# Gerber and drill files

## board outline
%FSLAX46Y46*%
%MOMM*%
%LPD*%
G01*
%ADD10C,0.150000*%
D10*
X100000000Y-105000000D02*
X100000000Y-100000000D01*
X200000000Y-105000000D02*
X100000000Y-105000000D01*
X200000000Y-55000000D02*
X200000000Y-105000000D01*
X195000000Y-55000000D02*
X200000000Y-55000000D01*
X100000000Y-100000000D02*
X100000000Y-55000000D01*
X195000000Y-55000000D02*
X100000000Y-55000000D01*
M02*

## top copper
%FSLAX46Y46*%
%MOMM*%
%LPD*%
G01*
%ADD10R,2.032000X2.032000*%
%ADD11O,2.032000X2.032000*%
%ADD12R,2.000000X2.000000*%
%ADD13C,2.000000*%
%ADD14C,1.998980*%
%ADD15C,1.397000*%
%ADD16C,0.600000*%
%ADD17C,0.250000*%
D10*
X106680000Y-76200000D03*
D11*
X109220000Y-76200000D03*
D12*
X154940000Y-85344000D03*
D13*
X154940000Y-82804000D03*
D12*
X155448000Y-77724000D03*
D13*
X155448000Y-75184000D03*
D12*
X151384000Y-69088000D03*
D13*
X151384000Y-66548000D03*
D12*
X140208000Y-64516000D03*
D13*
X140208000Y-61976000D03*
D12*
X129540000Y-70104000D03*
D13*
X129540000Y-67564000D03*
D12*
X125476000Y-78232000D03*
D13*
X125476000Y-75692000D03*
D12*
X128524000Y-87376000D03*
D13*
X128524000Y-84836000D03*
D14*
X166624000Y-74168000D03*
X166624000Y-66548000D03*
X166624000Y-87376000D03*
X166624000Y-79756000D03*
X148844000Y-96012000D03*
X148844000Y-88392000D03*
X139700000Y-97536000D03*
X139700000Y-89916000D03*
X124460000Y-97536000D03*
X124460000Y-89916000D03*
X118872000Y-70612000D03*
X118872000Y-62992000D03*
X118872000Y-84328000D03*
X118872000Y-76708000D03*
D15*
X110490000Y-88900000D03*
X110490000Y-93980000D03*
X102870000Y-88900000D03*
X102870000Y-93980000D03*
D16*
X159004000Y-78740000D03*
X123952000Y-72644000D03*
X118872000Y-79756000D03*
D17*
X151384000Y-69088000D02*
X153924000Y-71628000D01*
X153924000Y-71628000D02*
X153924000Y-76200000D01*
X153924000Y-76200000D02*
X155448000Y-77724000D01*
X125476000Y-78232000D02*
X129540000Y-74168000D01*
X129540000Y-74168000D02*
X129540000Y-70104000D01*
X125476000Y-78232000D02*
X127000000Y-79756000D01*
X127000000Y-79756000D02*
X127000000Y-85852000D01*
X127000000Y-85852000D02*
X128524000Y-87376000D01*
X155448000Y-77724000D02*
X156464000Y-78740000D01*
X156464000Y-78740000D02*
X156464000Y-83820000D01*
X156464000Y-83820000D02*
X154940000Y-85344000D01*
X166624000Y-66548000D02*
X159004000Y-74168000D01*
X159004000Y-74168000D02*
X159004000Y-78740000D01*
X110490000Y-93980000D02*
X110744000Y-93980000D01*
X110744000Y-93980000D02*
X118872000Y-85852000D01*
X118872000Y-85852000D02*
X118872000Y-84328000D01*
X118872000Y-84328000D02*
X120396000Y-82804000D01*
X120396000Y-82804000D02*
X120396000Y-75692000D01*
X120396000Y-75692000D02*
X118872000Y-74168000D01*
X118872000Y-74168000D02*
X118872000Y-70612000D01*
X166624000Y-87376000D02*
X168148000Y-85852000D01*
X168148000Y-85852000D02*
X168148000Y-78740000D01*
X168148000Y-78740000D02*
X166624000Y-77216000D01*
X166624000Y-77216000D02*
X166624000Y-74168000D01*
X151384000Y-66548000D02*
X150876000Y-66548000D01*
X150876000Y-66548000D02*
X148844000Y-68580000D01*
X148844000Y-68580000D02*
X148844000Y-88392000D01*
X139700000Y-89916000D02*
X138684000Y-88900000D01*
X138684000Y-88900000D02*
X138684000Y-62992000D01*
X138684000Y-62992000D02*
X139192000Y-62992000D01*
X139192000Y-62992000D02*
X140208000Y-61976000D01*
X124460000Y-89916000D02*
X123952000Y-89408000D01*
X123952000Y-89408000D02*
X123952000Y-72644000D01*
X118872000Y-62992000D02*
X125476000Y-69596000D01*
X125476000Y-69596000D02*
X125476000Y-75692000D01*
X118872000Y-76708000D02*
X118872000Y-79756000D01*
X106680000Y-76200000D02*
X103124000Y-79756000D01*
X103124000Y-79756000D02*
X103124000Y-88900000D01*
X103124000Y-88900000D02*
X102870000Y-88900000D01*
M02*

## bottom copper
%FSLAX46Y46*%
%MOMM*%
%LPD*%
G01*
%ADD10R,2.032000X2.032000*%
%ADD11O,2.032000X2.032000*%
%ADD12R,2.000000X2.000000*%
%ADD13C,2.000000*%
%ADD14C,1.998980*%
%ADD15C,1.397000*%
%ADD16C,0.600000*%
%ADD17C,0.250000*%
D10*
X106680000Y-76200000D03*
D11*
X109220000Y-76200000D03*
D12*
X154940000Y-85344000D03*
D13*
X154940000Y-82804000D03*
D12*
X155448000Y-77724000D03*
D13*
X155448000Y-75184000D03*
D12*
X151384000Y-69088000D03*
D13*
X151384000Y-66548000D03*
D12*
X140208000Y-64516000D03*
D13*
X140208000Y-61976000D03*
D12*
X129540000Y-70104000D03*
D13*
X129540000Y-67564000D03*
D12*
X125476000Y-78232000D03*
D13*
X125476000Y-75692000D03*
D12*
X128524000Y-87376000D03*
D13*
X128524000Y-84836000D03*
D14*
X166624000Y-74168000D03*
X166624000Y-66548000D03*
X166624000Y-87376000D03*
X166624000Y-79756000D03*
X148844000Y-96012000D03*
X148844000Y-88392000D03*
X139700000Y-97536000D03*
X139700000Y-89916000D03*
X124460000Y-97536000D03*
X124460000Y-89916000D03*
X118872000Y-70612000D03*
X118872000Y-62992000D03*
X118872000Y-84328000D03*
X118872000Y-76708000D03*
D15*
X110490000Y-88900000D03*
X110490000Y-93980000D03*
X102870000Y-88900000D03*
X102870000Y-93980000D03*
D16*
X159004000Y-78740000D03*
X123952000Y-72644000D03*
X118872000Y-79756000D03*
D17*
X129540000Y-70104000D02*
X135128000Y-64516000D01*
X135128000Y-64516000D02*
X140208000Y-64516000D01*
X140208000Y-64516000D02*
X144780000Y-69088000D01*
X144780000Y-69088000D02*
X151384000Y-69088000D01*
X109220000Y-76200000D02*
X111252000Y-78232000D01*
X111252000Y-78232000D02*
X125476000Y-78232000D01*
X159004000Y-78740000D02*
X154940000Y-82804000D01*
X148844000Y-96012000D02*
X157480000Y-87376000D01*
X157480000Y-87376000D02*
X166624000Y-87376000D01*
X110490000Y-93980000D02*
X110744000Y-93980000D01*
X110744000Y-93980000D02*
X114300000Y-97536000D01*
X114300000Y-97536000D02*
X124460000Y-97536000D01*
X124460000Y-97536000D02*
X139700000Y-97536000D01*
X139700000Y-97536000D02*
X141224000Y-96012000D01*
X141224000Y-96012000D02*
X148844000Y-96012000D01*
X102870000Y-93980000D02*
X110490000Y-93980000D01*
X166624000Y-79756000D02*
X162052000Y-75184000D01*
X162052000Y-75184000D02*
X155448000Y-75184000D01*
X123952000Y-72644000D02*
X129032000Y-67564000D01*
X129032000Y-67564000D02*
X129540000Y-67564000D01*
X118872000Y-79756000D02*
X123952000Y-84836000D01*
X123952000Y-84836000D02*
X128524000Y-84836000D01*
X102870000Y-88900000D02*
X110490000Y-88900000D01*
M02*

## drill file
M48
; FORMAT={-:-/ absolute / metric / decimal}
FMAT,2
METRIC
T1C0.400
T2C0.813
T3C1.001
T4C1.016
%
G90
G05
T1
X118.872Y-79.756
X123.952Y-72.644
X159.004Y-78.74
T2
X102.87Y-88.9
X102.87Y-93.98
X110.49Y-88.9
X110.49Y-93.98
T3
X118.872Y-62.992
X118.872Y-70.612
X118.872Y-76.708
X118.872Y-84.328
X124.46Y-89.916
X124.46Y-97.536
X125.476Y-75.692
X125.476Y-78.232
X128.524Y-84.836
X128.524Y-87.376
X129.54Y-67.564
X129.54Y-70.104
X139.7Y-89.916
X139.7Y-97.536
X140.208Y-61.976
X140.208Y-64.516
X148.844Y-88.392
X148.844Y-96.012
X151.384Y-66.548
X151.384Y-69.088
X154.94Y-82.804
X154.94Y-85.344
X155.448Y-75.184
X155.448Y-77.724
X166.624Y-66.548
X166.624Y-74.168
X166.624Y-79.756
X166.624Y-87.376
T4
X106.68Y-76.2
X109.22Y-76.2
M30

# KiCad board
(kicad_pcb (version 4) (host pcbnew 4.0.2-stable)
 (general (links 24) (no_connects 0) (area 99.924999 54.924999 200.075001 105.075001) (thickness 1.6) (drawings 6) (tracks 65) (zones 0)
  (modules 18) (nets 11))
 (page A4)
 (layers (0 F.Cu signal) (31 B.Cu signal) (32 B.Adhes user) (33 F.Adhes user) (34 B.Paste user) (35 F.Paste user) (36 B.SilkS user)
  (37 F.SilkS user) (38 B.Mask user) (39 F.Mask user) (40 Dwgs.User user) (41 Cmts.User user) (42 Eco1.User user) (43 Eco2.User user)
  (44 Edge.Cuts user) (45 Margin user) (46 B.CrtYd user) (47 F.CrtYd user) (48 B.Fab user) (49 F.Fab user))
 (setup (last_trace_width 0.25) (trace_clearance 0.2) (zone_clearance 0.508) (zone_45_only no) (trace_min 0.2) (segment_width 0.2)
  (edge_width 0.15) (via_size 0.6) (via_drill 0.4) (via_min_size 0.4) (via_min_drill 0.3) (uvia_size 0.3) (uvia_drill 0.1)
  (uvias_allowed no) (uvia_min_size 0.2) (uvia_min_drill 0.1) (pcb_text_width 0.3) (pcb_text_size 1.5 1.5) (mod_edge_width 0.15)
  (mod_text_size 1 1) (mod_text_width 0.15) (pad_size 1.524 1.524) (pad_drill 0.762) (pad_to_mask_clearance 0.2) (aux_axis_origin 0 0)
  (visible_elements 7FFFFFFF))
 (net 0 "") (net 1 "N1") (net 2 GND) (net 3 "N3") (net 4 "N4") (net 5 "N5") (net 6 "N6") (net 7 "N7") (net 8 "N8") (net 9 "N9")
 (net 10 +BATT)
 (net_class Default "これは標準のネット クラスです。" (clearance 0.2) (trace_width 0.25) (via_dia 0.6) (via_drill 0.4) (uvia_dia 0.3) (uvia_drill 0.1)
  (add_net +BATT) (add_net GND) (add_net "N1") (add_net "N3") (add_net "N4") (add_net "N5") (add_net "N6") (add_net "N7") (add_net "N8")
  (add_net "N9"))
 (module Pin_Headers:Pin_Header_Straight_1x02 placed (layer F.Cu) (at 106.68 76.2 90)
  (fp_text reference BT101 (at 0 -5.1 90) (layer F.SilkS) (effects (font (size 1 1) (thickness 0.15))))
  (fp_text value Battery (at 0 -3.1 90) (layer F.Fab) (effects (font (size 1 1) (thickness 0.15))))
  (pad 1 thru_hole rect (at 0 0 90) (size 2.032 2.032) (drill 1.016) (layers *.Cu *.Mask F.SilkS) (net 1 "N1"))
  (pad 2 thru_hole oval (at 0 2.54 90) (size 2.032 2.032) (drill 1.016) (layers *.Cu *.Mask F.SilkS) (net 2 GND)))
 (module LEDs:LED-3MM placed (layer F.Cu) (at 154.94 85.344 90)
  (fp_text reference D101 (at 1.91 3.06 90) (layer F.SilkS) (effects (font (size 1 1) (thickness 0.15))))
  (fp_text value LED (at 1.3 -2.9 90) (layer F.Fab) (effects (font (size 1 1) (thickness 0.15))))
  (pad 1 thru_hole rect (at 0 0 180) (size 2 2) (drill 1.00076) (layers *.Cu *.Mask F.SilkS) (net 2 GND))
  (pad 2 thru_hole circle (at 2.54 0 90) (size 2 2) (drill 1.00076) (layers *.Cu *.Mask F.SilkS) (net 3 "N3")))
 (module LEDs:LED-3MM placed (layer F.Cu) (at 155.448 77.724 90)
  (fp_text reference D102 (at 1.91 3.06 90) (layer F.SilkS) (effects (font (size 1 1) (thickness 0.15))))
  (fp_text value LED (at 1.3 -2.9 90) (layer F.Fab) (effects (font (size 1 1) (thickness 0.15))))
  (pad 1 thru_hole rect (at 0 0 180) (size 2 2) (drill 1.00076) (layers *.Cu *.Mask F.SilkS) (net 2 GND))
  (pad 2 thru_hole circle (at 2.54 0 90) (size 2 2) (drill 1.00076) (layers *.Cu *.Mask F.SilkS) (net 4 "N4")))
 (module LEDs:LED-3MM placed (layer F.Cu) (at 151.384 69.088 90)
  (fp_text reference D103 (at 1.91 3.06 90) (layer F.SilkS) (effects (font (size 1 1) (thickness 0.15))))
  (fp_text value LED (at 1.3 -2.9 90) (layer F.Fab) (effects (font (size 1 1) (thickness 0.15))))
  (pad 1 thru_hole rect (at 0 0 180) (size 2 2) (drill 1.00076) (layers *.Cu *.Mask F.SilkS) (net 2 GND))
  (pad 2 thru_hole circle (at 2.54 0 90) (size 2 2) (drill 1.00076) (layers *.Cu *.Mask F.SilkS) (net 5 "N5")))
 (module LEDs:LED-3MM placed (layer F.Cu) (at 140.208 64.516 90)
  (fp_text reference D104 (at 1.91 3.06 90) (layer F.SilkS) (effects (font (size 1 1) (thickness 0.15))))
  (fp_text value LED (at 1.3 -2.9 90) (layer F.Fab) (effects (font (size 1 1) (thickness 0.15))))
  (pad 1 thru_hole rect (at 0 0 180) (size 2 2) (drill 1.00076) (layers *.Cu *.Mask F.SilkS) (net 2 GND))
  (pad 2 thru_hole circle (at 2.54 0 90) (size 2 2) (drill 1.00076) (layers *.Cu *.Mask F.SilkS) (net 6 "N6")))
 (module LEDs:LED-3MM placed (layer F.Cu) (at 129.54 70.104 90)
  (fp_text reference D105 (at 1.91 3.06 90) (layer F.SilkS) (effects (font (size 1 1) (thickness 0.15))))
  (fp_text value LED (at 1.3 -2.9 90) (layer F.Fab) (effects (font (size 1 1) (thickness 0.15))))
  (pad 1 thru_hole rect (at 0 0 180) (size 2 2) (drill 1.00076) (layers *.Cu *.Mask F.SilkS) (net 2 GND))
  (pad 2 thru_hole circle (at 2.54 0 90) (size 2 2) (drill 1.00076) (layers *.Cu *.Mask F.SilkS) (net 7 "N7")))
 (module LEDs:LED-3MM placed (layer F.Cu) (at 125.476 78.232 90)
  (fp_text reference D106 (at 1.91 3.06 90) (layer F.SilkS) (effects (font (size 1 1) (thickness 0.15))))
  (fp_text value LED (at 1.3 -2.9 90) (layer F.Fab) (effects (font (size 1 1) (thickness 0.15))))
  (pad 1 thru_hole rect (at 0 0 180) (size 2 2) (drill 1.00076) (layers *.Cu *.Mask F.SilkS) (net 2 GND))
  (pad 2 thru_hole circle (at 2.54 0 90) (size 2 2) (drill 1.00076) (layers *.Cu *.Mask F.SilkS) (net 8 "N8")))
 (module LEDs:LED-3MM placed (layer F.Cu) (at 128.524 87.376 90)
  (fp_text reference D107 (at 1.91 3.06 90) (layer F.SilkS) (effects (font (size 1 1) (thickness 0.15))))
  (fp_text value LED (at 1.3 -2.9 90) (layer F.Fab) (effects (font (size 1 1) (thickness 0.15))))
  (pad 1 thru_hole rect (at 0 0 180) (size 2 2) (drill 1.00076) (layers *.Cu *.Mask F.SilkS) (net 2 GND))
  (pad 2 thru_hole circle (at 2.54 0 90) (size 2 2) (drill 1.00076) (layers *.Cu *.Mask F.SilkS) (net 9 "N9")))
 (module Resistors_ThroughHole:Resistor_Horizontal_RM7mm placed (layer F.Cu) (at 166.624 74.168 90)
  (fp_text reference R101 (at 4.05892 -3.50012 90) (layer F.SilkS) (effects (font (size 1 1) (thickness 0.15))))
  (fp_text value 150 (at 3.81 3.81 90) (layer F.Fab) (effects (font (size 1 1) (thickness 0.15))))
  (pad 1 thru_hole circle (at 0 0 90) (size 1.99898 1.99898) (drill 1.00076) (layers *.Cu *.SilkS *.Mask) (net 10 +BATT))
  (pad 2 thru_hole circle (at 7.62 0 90) (size 1.99898 1.99898) (drill 1.00076) (layers *.Cu *.SilkS *.Mask) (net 3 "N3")))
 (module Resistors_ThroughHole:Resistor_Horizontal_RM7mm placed (layer F.Cu) (at 166.624 87.376 90)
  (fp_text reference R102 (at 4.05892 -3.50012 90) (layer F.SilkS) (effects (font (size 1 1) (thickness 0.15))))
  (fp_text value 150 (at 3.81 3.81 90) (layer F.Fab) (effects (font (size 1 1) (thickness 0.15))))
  (pad 1 thru_hole circle (at 0 0 90) (size 1.99898 1.99898) (drill 1.00076) (layers *.Cu *.SilkS *.Mask) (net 10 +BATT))
  (pad 2 thru_hole circle (at 7.62 0 90) (size 1.99898 1.99898) (drill 1.00076) (layers *.Cu *.SilkS *.Mask) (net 4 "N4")))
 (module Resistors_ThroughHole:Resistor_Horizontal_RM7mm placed (layer F.Cu) (at 148.844 96.012 90)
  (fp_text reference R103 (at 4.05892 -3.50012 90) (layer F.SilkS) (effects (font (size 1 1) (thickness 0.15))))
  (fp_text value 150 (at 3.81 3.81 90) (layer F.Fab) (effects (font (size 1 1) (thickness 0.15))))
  (pad 1 thru_hole circle (at 0 0 90) (size 1.99898 1.99898) (drill 1.00076) (layers *.Cu *.SilkS *.Mask) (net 10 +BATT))
  (pad 2 thru_hole circle (at 7.62 0 90) (size 1.99898 1.99898) (drill 1.00076) (layers *.Cu *.SilkS *.Mask) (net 5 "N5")))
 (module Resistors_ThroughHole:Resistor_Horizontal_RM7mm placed (layer F.Cu) (at 139.7 97.536 90)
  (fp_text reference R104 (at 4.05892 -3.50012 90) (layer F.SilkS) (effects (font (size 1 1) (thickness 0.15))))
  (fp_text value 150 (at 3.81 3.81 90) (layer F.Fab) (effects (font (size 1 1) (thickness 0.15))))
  (pad 1 thru_hole circle (at 0 0 90) (size 1.99898 1.99898) (drill 1.00076) (layers *.Cu *.SilkS *.Mask) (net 10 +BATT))
  (pad 2 thru_hole circle (at 7.62 0 90) (size 1.99898 1.99898) (drill 1.00076) (layers *.Cu *.SilkS *.Mask) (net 6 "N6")))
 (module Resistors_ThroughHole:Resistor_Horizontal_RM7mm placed (layer F.Cu) (at 124.46 97.536 90)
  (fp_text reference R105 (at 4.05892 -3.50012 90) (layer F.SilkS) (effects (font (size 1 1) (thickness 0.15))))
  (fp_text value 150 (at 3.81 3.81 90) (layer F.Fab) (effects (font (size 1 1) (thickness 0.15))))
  (pad 1 thru_hole circle (at 0 0 90) (size 1.99898 1.99898) (drill 1.00076) (layers *.Cu *.SilkS *.Mask) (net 10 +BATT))
  (pad 2 thru_hole circle (at 7.62 0 90) (size 1.99898 1.99898) (drill 1.00076) (layers *.Cu *.SilkS *.Mask) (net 7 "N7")))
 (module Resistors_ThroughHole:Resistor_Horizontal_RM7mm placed (layer F.Cu) (at 118.872 70.612 90)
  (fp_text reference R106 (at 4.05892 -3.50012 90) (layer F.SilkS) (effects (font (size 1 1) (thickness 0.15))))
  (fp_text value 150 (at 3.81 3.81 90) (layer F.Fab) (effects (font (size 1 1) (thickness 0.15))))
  (pad 1 thru_hole circle (at 0 0 90) (size 1.99898 1.99898) (drill 1.00076) (layers *.Cu *.SilkS *.Mask) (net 10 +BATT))
  (pad 2 thru_hole circle (at 7.62 0 90) (size 1.99898 1.99898) (drill 1.00076) (layers *.Cu *.SilkS *.Mask) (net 8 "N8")))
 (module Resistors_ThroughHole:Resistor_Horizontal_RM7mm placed (layer F.Cu) (at 118.872 84.328 90)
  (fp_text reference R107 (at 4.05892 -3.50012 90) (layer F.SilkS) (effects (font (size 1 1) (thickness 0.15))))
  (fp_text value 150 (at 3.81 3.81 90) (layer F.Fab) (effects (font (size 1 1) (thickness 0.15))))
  (pad 1 thru_hole circle (at 0 0 90) (size 1.99898 1.99898) (drill 1.00076) (layers *.Cu *.SilkS *.Mask) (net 10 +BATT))
  (pad 2 thru_hole circle (at 7.62 0 90) (size 1.99898 1.99898) (drill 1.00076) (layers *.Cu *.SilkS *.Mask) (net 9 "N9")))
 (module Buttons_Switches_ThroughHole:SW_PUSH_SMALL (layer F.Cu) (at 106.68 91.44)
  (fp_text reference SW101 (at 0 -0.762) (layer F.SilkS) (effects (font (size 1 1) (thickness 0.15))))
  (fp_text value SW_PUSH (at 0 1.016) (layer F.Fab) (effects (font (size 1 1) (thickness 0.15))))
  (pad 1 thru_hole circle (at 3.81 -2.54) (size 1.397 1.397) (drill 0.8128) (layers *.Cu *.Mask F.SilkS) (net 1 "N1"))
  (pad 2 thru_hole circle (at 3.81 2.54) (size 1.397 1.397) (drill 0.8128) (layers *.Cu *.Mask F.SilkS) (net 10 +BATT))
  (pad 1 thru_hole circle (at -3.81 -2.54) (size 1.397 1.397) (drill 0.8128) (layers *.Cu *.Mask F.SilkS) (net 1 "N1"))
  (pad 2 thru_hole circle (at -3.81 2.54) (size 1.397 1.397) (drill 0.8128) (layers *.Cu *.Mask F.SilkS) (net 10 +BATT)))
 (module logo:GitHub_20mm (layer F.Cu) (at 139.7 77.724)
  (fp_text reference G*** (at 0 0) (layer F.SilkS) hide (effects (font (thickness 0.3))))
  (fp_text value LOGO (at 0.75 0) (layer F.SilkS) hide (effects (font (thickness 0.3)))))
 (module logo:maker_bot (layer F.Cu) (at 181.864 75.692)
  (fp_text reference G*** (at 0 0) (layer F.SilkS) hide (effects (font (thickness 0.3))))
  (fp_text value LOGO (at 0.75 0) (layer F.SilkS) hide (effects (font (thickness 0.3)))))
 (gr_line (start 100 105) (end 100 100) (angle 90) (layer Edge.Cuts) (width 0.15))
 (gr_line (start 200 105) (end 100 105) (angle 90) (layer Edge.Cuts) (width 0.15))
 (gr_line (start 200 55) (end 200 105) (angle 90) (layer Edge.Cuts) (width 0.15))
 (gr_line (start 195 55) (end 200 55) (angle 90) (layer Edge.Cuts) (width 0.15))
 (gr_line (start 100 100) (end 100 55) (angle 90) (layer Edge.Cuts) (width 0.15))
 (gr_line (start 195 55) (end 100 55) (angle 90) (layer Edge.Cuts) (width 0.15))
 (segment (start 129.54 70.104) (end 135.128 64.516) (width 0.25) (layer B.Cu) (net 2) (status 80000))
 (segment (start 135.128 64.516) (end 140.208 64.516) (width 0.25) (layer B.Cu) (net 2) (status 80000))
 (segment (start 140.208 64.516) (end 144.78 69.088) (width 0.25) (layer B.Cu) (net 2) (status 80000))
 (segment (start 144.78 69.088) (end 151.384 69.088) (width 0.25) (layer B.Cu) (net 2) (status 80000))
 (segment (start 151.384 69.088) (end 153.924 71.628) (width 0.25) (layer F.Cu) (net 2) (status 80000))
 (segment (start 153.924 71.628) (end 153.924 76.2) (width 0.25) (layer F.Cu) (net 2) (status 80000))
 (segment (start 153.924 76.2) (end 155.448 77.724) (width 0.25) (layer F.Cu) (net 2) (status 80000))
 (segment (start 125.476 78.232) (end 129.54 74.168) (width 0.25) (layer F.Cu) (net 2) (status 80000))
 (segment (start 129.54 74.168) (end 129.54 70.104) (width 0.25) (layer F.Cu) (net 2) (status 80000))
 (segment (start 109.22 76.2) (end 111.252 78.232) (width 0.25) (layer B.Cu) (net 2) (status 80000))
 (segment (start 111.252 78.232) (end 125.476 78.232) (width 0.25) (layer B.Cu) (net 2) (status 80000))
 (segment (start 125.476 78.232) (end 127 79.756) (width 0.25) (layer F.Cu) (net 2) (status 80000))
 (segment (start 127 79.756) (end 127 85.852) (width 0.25) (layer F.Cu) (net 2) (status 80000))
 (segment (start 127 85.852) (end 128.524 87.376) (width 0.25) (layer F.Cu) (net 2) (status 80000))
 (segment (start 155.448 77.724) (end 156.464 78.74) (width 0.25) (layer F.Cu) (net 2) (status 80000))
 (segment (start 156.464 78.74) (end 156.464 83.82) (width 0.25) (layer F.Cu) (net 2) (status 80000))
 (segment (start 156.464 83.82) (end 154.94 85.344) (width 0.25) (layer F.Cu) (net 2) (status 80000))
 (segment (start 166.624 66.548) (end 159.004 74.168) (width 0.25) (layer F.Cu) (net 3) (status 80000))
 (segment (start 159.004 74.168) (end 159.004 78.74) (width 0.25) (layer F.Cu) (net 3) (status 80000))
 (via (at 159.004 78.74) (size 0.6) (layers F.Cu B.Cu) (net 3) (status 80000))
 (segment (start 159.004 78.74) (end 154.94 82.804) (width 0.25) (layer B.Cu) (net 3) (status 80000))
 (segment (start 148.844 96.012) (end 157.48 87.376) (width 0.25) (layer B.Cu) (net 10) (status 80000))
 (segment (start 157.48 87.376) (end 166.624 87.376) (width 0.25) (layer B.Cu) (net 10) (status 80000))
 (segment (start 110.49 93.98) (end 110.744 93.98) (width 0.25) (layer F.Cu) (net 10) (status 80000))
 (segment (start 110.744 93.98) (end 118.872 85.852) (width 0.25) (layer F.Cu) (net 10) (status 80000))
 (segment (start 118.872 85.852) (end 118.872 84.328) (width 0.25) (layer F.Cu) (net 10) (status 80000))
 (segment (start 110.49 93.98) (end 110.744 93.98) (width 0.25) (layer B.Cu) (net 10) (status 80000))
 (segment (start 110.744 93.98) (end 114.3 97.536) (width 0.25) (layer B.Cu) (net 10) (status 80000))
 (segment (start 114.3 97.536) (end 124.46 97.536) (width 0.25) (layer B.Cu) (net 10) (status 80000))
 (segment (start 124.46 97.536) (end 139.7 97.536) (width 0.25) (layer B.Cu) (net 10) (status 80000))
 (segment (start 139.7 97.536) (end 141.224 96.012) (width 0.25) (layer B.Cu) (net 10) (status 80000))
 (segment (start 141.224 96.012) (end 148.844 96.012) (width 0.25) (layer B.Cu) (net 10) (status 80000))
 (segment (start 118.872 84.328) (end 120.396 82.804) (width 0.25) (layer F.Cu) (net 10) (status 80000))
 (segment (start 120.396 82.804) (end 120.396 75.692) (width 0.25) (layer F.Cu) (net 10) (status 80000))
 (segment (start 120.396 75.692) (end 118.872 74.168) (width 0.25) (layer F.Cu) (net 10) (status 80000))
 (segment (start 118.872 74.168) (end 118.872 70.612) (width 0.25) (layer F.Cu) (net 10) (status 80000))
 (segment (start 166.624 87.376) (end 168.148 85.852) (width 0.25) (layer F.Cu) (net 10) (status 80000))
 (segment (start 168.148 85.852) (end 168.148 78.74) (width 0.25) (layer F.Cu) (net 10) (status 80000))
 (segment (start 168.148 78.74) (end 166.624 77.216) (width 0.25) (layer F.Cu) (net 10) (status 80000))
 (segment (start 166.624 77.216) (end 166.624 74.168) (width 0.25) (layer F.Cu) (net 10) (status 80000))
 (segment (start 102.87 93.98) (end 110.49 93.98) (width 0.25) (layer B.Cu) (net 10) (status 80000))
 (segment (start 166.624 79.756) (end 162.052 75.184) (width 0.25) (layer B.Cu) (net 4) (status 80000))
 (segment (start 162.052 75.184) (end 155.448 75.184) (width 0.25) (layer B.Cu) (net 4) (status 80000))
 (segment (start 151.384 66.548) (end 150.876 66.548) (width 0.25) (layer F.Cu) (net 5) (status 80000))
 (segment (start 150.876 66.548) (end 148.844 68.58) (width 0.25) (layer F.Cu) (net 5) (status 80000))
 (segment (start 148.844 68.58) (end 148.844 88.392) (width 0.25) (layer F.Cu) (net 5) (status 80000))
 (segment (start 139.7 89.916) (end 138.684 88.9) (width 0.25) (layer F.Cu) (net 6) (status 80000))
 (segment (start 138.684 88.9) (end 138.684 62.992) (width 0.25) (layer F.Cu) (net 6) (status 80000))
 (segment (start 138.684 62.992) (end 139.192 62.992) (width 0.25) (layer F.Cu) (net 6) (status 80000))
 (segment (start 139.192 62.992) (end 140.208 61.976) (width 0.25) (layer F.Cu) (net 6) (status 80000))
 (segment (start 124.46 89.916) (end 123.952 89.408) (width 0.25) (layer F.Cu) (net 7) (status 80000))
 (segment (start 123.952 89.408) (end 123.952 72.644) (width 0.25) (layer F.Cu) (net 7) (status 80000))
 (via (at 123.952 72.644) (size 0.6) (layers F.Cu B.Cu) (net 7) (status 80000))
 (segment (start 123.952 72.644) (end 129.032 67.564) (width 0.25) (layer B.Cu) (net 7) (status 80000))
 (segment (start 129.032 67.564) (end 129.54 67.564) (width 0.25) (layer B.Cu) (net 7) (status 80000))
 (segment (start 118.872 62.992) (end 125.476 69.596) (width 0.25) (layer F.Cu) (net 8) (status 80000))
 (segment (start 125.476 69.596) (end 125.476 75.692) (width 0.25) (layer F.Cu) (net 8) (status 80000))
 (segment (start 118.872 76.708) (end 118.872 79.756) (width 0.25) (layer F.Cu) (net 9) (status 80000))
 (via (at 118.872 79.756) (size 0.6) (layers F.Cu B.Cu) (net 9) (status 80000))
 (segment (start 118.872 79.756) (end 123.952 84.836) (width 0.25) (layer B.Cu) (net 9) (status 80000))
 (segment (start 123.952 84.836) (end 128.524 84.836) (width 0.25) (layer B.Cu) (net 9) (status 80000))
 (segment (start 106.68 76.2) (end 103.124 79.756) (width 0.25) (layer F.Cu) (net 1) (status 80000))
 (segment (start 103.124 79.756) (end 103.124 88.9) (width 0.25) (layer F.Cu) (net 1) (status 80000))
 (segment (start 103.124 88.9) (end 102.87 88.9) (width 0.25) (layer F.Cu) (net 1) (status 80000))
 (segment (start 102.87 88.9) (end 110.49 88.9) (width 0.25) (layer B.Cu) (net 1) (status 80000)))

